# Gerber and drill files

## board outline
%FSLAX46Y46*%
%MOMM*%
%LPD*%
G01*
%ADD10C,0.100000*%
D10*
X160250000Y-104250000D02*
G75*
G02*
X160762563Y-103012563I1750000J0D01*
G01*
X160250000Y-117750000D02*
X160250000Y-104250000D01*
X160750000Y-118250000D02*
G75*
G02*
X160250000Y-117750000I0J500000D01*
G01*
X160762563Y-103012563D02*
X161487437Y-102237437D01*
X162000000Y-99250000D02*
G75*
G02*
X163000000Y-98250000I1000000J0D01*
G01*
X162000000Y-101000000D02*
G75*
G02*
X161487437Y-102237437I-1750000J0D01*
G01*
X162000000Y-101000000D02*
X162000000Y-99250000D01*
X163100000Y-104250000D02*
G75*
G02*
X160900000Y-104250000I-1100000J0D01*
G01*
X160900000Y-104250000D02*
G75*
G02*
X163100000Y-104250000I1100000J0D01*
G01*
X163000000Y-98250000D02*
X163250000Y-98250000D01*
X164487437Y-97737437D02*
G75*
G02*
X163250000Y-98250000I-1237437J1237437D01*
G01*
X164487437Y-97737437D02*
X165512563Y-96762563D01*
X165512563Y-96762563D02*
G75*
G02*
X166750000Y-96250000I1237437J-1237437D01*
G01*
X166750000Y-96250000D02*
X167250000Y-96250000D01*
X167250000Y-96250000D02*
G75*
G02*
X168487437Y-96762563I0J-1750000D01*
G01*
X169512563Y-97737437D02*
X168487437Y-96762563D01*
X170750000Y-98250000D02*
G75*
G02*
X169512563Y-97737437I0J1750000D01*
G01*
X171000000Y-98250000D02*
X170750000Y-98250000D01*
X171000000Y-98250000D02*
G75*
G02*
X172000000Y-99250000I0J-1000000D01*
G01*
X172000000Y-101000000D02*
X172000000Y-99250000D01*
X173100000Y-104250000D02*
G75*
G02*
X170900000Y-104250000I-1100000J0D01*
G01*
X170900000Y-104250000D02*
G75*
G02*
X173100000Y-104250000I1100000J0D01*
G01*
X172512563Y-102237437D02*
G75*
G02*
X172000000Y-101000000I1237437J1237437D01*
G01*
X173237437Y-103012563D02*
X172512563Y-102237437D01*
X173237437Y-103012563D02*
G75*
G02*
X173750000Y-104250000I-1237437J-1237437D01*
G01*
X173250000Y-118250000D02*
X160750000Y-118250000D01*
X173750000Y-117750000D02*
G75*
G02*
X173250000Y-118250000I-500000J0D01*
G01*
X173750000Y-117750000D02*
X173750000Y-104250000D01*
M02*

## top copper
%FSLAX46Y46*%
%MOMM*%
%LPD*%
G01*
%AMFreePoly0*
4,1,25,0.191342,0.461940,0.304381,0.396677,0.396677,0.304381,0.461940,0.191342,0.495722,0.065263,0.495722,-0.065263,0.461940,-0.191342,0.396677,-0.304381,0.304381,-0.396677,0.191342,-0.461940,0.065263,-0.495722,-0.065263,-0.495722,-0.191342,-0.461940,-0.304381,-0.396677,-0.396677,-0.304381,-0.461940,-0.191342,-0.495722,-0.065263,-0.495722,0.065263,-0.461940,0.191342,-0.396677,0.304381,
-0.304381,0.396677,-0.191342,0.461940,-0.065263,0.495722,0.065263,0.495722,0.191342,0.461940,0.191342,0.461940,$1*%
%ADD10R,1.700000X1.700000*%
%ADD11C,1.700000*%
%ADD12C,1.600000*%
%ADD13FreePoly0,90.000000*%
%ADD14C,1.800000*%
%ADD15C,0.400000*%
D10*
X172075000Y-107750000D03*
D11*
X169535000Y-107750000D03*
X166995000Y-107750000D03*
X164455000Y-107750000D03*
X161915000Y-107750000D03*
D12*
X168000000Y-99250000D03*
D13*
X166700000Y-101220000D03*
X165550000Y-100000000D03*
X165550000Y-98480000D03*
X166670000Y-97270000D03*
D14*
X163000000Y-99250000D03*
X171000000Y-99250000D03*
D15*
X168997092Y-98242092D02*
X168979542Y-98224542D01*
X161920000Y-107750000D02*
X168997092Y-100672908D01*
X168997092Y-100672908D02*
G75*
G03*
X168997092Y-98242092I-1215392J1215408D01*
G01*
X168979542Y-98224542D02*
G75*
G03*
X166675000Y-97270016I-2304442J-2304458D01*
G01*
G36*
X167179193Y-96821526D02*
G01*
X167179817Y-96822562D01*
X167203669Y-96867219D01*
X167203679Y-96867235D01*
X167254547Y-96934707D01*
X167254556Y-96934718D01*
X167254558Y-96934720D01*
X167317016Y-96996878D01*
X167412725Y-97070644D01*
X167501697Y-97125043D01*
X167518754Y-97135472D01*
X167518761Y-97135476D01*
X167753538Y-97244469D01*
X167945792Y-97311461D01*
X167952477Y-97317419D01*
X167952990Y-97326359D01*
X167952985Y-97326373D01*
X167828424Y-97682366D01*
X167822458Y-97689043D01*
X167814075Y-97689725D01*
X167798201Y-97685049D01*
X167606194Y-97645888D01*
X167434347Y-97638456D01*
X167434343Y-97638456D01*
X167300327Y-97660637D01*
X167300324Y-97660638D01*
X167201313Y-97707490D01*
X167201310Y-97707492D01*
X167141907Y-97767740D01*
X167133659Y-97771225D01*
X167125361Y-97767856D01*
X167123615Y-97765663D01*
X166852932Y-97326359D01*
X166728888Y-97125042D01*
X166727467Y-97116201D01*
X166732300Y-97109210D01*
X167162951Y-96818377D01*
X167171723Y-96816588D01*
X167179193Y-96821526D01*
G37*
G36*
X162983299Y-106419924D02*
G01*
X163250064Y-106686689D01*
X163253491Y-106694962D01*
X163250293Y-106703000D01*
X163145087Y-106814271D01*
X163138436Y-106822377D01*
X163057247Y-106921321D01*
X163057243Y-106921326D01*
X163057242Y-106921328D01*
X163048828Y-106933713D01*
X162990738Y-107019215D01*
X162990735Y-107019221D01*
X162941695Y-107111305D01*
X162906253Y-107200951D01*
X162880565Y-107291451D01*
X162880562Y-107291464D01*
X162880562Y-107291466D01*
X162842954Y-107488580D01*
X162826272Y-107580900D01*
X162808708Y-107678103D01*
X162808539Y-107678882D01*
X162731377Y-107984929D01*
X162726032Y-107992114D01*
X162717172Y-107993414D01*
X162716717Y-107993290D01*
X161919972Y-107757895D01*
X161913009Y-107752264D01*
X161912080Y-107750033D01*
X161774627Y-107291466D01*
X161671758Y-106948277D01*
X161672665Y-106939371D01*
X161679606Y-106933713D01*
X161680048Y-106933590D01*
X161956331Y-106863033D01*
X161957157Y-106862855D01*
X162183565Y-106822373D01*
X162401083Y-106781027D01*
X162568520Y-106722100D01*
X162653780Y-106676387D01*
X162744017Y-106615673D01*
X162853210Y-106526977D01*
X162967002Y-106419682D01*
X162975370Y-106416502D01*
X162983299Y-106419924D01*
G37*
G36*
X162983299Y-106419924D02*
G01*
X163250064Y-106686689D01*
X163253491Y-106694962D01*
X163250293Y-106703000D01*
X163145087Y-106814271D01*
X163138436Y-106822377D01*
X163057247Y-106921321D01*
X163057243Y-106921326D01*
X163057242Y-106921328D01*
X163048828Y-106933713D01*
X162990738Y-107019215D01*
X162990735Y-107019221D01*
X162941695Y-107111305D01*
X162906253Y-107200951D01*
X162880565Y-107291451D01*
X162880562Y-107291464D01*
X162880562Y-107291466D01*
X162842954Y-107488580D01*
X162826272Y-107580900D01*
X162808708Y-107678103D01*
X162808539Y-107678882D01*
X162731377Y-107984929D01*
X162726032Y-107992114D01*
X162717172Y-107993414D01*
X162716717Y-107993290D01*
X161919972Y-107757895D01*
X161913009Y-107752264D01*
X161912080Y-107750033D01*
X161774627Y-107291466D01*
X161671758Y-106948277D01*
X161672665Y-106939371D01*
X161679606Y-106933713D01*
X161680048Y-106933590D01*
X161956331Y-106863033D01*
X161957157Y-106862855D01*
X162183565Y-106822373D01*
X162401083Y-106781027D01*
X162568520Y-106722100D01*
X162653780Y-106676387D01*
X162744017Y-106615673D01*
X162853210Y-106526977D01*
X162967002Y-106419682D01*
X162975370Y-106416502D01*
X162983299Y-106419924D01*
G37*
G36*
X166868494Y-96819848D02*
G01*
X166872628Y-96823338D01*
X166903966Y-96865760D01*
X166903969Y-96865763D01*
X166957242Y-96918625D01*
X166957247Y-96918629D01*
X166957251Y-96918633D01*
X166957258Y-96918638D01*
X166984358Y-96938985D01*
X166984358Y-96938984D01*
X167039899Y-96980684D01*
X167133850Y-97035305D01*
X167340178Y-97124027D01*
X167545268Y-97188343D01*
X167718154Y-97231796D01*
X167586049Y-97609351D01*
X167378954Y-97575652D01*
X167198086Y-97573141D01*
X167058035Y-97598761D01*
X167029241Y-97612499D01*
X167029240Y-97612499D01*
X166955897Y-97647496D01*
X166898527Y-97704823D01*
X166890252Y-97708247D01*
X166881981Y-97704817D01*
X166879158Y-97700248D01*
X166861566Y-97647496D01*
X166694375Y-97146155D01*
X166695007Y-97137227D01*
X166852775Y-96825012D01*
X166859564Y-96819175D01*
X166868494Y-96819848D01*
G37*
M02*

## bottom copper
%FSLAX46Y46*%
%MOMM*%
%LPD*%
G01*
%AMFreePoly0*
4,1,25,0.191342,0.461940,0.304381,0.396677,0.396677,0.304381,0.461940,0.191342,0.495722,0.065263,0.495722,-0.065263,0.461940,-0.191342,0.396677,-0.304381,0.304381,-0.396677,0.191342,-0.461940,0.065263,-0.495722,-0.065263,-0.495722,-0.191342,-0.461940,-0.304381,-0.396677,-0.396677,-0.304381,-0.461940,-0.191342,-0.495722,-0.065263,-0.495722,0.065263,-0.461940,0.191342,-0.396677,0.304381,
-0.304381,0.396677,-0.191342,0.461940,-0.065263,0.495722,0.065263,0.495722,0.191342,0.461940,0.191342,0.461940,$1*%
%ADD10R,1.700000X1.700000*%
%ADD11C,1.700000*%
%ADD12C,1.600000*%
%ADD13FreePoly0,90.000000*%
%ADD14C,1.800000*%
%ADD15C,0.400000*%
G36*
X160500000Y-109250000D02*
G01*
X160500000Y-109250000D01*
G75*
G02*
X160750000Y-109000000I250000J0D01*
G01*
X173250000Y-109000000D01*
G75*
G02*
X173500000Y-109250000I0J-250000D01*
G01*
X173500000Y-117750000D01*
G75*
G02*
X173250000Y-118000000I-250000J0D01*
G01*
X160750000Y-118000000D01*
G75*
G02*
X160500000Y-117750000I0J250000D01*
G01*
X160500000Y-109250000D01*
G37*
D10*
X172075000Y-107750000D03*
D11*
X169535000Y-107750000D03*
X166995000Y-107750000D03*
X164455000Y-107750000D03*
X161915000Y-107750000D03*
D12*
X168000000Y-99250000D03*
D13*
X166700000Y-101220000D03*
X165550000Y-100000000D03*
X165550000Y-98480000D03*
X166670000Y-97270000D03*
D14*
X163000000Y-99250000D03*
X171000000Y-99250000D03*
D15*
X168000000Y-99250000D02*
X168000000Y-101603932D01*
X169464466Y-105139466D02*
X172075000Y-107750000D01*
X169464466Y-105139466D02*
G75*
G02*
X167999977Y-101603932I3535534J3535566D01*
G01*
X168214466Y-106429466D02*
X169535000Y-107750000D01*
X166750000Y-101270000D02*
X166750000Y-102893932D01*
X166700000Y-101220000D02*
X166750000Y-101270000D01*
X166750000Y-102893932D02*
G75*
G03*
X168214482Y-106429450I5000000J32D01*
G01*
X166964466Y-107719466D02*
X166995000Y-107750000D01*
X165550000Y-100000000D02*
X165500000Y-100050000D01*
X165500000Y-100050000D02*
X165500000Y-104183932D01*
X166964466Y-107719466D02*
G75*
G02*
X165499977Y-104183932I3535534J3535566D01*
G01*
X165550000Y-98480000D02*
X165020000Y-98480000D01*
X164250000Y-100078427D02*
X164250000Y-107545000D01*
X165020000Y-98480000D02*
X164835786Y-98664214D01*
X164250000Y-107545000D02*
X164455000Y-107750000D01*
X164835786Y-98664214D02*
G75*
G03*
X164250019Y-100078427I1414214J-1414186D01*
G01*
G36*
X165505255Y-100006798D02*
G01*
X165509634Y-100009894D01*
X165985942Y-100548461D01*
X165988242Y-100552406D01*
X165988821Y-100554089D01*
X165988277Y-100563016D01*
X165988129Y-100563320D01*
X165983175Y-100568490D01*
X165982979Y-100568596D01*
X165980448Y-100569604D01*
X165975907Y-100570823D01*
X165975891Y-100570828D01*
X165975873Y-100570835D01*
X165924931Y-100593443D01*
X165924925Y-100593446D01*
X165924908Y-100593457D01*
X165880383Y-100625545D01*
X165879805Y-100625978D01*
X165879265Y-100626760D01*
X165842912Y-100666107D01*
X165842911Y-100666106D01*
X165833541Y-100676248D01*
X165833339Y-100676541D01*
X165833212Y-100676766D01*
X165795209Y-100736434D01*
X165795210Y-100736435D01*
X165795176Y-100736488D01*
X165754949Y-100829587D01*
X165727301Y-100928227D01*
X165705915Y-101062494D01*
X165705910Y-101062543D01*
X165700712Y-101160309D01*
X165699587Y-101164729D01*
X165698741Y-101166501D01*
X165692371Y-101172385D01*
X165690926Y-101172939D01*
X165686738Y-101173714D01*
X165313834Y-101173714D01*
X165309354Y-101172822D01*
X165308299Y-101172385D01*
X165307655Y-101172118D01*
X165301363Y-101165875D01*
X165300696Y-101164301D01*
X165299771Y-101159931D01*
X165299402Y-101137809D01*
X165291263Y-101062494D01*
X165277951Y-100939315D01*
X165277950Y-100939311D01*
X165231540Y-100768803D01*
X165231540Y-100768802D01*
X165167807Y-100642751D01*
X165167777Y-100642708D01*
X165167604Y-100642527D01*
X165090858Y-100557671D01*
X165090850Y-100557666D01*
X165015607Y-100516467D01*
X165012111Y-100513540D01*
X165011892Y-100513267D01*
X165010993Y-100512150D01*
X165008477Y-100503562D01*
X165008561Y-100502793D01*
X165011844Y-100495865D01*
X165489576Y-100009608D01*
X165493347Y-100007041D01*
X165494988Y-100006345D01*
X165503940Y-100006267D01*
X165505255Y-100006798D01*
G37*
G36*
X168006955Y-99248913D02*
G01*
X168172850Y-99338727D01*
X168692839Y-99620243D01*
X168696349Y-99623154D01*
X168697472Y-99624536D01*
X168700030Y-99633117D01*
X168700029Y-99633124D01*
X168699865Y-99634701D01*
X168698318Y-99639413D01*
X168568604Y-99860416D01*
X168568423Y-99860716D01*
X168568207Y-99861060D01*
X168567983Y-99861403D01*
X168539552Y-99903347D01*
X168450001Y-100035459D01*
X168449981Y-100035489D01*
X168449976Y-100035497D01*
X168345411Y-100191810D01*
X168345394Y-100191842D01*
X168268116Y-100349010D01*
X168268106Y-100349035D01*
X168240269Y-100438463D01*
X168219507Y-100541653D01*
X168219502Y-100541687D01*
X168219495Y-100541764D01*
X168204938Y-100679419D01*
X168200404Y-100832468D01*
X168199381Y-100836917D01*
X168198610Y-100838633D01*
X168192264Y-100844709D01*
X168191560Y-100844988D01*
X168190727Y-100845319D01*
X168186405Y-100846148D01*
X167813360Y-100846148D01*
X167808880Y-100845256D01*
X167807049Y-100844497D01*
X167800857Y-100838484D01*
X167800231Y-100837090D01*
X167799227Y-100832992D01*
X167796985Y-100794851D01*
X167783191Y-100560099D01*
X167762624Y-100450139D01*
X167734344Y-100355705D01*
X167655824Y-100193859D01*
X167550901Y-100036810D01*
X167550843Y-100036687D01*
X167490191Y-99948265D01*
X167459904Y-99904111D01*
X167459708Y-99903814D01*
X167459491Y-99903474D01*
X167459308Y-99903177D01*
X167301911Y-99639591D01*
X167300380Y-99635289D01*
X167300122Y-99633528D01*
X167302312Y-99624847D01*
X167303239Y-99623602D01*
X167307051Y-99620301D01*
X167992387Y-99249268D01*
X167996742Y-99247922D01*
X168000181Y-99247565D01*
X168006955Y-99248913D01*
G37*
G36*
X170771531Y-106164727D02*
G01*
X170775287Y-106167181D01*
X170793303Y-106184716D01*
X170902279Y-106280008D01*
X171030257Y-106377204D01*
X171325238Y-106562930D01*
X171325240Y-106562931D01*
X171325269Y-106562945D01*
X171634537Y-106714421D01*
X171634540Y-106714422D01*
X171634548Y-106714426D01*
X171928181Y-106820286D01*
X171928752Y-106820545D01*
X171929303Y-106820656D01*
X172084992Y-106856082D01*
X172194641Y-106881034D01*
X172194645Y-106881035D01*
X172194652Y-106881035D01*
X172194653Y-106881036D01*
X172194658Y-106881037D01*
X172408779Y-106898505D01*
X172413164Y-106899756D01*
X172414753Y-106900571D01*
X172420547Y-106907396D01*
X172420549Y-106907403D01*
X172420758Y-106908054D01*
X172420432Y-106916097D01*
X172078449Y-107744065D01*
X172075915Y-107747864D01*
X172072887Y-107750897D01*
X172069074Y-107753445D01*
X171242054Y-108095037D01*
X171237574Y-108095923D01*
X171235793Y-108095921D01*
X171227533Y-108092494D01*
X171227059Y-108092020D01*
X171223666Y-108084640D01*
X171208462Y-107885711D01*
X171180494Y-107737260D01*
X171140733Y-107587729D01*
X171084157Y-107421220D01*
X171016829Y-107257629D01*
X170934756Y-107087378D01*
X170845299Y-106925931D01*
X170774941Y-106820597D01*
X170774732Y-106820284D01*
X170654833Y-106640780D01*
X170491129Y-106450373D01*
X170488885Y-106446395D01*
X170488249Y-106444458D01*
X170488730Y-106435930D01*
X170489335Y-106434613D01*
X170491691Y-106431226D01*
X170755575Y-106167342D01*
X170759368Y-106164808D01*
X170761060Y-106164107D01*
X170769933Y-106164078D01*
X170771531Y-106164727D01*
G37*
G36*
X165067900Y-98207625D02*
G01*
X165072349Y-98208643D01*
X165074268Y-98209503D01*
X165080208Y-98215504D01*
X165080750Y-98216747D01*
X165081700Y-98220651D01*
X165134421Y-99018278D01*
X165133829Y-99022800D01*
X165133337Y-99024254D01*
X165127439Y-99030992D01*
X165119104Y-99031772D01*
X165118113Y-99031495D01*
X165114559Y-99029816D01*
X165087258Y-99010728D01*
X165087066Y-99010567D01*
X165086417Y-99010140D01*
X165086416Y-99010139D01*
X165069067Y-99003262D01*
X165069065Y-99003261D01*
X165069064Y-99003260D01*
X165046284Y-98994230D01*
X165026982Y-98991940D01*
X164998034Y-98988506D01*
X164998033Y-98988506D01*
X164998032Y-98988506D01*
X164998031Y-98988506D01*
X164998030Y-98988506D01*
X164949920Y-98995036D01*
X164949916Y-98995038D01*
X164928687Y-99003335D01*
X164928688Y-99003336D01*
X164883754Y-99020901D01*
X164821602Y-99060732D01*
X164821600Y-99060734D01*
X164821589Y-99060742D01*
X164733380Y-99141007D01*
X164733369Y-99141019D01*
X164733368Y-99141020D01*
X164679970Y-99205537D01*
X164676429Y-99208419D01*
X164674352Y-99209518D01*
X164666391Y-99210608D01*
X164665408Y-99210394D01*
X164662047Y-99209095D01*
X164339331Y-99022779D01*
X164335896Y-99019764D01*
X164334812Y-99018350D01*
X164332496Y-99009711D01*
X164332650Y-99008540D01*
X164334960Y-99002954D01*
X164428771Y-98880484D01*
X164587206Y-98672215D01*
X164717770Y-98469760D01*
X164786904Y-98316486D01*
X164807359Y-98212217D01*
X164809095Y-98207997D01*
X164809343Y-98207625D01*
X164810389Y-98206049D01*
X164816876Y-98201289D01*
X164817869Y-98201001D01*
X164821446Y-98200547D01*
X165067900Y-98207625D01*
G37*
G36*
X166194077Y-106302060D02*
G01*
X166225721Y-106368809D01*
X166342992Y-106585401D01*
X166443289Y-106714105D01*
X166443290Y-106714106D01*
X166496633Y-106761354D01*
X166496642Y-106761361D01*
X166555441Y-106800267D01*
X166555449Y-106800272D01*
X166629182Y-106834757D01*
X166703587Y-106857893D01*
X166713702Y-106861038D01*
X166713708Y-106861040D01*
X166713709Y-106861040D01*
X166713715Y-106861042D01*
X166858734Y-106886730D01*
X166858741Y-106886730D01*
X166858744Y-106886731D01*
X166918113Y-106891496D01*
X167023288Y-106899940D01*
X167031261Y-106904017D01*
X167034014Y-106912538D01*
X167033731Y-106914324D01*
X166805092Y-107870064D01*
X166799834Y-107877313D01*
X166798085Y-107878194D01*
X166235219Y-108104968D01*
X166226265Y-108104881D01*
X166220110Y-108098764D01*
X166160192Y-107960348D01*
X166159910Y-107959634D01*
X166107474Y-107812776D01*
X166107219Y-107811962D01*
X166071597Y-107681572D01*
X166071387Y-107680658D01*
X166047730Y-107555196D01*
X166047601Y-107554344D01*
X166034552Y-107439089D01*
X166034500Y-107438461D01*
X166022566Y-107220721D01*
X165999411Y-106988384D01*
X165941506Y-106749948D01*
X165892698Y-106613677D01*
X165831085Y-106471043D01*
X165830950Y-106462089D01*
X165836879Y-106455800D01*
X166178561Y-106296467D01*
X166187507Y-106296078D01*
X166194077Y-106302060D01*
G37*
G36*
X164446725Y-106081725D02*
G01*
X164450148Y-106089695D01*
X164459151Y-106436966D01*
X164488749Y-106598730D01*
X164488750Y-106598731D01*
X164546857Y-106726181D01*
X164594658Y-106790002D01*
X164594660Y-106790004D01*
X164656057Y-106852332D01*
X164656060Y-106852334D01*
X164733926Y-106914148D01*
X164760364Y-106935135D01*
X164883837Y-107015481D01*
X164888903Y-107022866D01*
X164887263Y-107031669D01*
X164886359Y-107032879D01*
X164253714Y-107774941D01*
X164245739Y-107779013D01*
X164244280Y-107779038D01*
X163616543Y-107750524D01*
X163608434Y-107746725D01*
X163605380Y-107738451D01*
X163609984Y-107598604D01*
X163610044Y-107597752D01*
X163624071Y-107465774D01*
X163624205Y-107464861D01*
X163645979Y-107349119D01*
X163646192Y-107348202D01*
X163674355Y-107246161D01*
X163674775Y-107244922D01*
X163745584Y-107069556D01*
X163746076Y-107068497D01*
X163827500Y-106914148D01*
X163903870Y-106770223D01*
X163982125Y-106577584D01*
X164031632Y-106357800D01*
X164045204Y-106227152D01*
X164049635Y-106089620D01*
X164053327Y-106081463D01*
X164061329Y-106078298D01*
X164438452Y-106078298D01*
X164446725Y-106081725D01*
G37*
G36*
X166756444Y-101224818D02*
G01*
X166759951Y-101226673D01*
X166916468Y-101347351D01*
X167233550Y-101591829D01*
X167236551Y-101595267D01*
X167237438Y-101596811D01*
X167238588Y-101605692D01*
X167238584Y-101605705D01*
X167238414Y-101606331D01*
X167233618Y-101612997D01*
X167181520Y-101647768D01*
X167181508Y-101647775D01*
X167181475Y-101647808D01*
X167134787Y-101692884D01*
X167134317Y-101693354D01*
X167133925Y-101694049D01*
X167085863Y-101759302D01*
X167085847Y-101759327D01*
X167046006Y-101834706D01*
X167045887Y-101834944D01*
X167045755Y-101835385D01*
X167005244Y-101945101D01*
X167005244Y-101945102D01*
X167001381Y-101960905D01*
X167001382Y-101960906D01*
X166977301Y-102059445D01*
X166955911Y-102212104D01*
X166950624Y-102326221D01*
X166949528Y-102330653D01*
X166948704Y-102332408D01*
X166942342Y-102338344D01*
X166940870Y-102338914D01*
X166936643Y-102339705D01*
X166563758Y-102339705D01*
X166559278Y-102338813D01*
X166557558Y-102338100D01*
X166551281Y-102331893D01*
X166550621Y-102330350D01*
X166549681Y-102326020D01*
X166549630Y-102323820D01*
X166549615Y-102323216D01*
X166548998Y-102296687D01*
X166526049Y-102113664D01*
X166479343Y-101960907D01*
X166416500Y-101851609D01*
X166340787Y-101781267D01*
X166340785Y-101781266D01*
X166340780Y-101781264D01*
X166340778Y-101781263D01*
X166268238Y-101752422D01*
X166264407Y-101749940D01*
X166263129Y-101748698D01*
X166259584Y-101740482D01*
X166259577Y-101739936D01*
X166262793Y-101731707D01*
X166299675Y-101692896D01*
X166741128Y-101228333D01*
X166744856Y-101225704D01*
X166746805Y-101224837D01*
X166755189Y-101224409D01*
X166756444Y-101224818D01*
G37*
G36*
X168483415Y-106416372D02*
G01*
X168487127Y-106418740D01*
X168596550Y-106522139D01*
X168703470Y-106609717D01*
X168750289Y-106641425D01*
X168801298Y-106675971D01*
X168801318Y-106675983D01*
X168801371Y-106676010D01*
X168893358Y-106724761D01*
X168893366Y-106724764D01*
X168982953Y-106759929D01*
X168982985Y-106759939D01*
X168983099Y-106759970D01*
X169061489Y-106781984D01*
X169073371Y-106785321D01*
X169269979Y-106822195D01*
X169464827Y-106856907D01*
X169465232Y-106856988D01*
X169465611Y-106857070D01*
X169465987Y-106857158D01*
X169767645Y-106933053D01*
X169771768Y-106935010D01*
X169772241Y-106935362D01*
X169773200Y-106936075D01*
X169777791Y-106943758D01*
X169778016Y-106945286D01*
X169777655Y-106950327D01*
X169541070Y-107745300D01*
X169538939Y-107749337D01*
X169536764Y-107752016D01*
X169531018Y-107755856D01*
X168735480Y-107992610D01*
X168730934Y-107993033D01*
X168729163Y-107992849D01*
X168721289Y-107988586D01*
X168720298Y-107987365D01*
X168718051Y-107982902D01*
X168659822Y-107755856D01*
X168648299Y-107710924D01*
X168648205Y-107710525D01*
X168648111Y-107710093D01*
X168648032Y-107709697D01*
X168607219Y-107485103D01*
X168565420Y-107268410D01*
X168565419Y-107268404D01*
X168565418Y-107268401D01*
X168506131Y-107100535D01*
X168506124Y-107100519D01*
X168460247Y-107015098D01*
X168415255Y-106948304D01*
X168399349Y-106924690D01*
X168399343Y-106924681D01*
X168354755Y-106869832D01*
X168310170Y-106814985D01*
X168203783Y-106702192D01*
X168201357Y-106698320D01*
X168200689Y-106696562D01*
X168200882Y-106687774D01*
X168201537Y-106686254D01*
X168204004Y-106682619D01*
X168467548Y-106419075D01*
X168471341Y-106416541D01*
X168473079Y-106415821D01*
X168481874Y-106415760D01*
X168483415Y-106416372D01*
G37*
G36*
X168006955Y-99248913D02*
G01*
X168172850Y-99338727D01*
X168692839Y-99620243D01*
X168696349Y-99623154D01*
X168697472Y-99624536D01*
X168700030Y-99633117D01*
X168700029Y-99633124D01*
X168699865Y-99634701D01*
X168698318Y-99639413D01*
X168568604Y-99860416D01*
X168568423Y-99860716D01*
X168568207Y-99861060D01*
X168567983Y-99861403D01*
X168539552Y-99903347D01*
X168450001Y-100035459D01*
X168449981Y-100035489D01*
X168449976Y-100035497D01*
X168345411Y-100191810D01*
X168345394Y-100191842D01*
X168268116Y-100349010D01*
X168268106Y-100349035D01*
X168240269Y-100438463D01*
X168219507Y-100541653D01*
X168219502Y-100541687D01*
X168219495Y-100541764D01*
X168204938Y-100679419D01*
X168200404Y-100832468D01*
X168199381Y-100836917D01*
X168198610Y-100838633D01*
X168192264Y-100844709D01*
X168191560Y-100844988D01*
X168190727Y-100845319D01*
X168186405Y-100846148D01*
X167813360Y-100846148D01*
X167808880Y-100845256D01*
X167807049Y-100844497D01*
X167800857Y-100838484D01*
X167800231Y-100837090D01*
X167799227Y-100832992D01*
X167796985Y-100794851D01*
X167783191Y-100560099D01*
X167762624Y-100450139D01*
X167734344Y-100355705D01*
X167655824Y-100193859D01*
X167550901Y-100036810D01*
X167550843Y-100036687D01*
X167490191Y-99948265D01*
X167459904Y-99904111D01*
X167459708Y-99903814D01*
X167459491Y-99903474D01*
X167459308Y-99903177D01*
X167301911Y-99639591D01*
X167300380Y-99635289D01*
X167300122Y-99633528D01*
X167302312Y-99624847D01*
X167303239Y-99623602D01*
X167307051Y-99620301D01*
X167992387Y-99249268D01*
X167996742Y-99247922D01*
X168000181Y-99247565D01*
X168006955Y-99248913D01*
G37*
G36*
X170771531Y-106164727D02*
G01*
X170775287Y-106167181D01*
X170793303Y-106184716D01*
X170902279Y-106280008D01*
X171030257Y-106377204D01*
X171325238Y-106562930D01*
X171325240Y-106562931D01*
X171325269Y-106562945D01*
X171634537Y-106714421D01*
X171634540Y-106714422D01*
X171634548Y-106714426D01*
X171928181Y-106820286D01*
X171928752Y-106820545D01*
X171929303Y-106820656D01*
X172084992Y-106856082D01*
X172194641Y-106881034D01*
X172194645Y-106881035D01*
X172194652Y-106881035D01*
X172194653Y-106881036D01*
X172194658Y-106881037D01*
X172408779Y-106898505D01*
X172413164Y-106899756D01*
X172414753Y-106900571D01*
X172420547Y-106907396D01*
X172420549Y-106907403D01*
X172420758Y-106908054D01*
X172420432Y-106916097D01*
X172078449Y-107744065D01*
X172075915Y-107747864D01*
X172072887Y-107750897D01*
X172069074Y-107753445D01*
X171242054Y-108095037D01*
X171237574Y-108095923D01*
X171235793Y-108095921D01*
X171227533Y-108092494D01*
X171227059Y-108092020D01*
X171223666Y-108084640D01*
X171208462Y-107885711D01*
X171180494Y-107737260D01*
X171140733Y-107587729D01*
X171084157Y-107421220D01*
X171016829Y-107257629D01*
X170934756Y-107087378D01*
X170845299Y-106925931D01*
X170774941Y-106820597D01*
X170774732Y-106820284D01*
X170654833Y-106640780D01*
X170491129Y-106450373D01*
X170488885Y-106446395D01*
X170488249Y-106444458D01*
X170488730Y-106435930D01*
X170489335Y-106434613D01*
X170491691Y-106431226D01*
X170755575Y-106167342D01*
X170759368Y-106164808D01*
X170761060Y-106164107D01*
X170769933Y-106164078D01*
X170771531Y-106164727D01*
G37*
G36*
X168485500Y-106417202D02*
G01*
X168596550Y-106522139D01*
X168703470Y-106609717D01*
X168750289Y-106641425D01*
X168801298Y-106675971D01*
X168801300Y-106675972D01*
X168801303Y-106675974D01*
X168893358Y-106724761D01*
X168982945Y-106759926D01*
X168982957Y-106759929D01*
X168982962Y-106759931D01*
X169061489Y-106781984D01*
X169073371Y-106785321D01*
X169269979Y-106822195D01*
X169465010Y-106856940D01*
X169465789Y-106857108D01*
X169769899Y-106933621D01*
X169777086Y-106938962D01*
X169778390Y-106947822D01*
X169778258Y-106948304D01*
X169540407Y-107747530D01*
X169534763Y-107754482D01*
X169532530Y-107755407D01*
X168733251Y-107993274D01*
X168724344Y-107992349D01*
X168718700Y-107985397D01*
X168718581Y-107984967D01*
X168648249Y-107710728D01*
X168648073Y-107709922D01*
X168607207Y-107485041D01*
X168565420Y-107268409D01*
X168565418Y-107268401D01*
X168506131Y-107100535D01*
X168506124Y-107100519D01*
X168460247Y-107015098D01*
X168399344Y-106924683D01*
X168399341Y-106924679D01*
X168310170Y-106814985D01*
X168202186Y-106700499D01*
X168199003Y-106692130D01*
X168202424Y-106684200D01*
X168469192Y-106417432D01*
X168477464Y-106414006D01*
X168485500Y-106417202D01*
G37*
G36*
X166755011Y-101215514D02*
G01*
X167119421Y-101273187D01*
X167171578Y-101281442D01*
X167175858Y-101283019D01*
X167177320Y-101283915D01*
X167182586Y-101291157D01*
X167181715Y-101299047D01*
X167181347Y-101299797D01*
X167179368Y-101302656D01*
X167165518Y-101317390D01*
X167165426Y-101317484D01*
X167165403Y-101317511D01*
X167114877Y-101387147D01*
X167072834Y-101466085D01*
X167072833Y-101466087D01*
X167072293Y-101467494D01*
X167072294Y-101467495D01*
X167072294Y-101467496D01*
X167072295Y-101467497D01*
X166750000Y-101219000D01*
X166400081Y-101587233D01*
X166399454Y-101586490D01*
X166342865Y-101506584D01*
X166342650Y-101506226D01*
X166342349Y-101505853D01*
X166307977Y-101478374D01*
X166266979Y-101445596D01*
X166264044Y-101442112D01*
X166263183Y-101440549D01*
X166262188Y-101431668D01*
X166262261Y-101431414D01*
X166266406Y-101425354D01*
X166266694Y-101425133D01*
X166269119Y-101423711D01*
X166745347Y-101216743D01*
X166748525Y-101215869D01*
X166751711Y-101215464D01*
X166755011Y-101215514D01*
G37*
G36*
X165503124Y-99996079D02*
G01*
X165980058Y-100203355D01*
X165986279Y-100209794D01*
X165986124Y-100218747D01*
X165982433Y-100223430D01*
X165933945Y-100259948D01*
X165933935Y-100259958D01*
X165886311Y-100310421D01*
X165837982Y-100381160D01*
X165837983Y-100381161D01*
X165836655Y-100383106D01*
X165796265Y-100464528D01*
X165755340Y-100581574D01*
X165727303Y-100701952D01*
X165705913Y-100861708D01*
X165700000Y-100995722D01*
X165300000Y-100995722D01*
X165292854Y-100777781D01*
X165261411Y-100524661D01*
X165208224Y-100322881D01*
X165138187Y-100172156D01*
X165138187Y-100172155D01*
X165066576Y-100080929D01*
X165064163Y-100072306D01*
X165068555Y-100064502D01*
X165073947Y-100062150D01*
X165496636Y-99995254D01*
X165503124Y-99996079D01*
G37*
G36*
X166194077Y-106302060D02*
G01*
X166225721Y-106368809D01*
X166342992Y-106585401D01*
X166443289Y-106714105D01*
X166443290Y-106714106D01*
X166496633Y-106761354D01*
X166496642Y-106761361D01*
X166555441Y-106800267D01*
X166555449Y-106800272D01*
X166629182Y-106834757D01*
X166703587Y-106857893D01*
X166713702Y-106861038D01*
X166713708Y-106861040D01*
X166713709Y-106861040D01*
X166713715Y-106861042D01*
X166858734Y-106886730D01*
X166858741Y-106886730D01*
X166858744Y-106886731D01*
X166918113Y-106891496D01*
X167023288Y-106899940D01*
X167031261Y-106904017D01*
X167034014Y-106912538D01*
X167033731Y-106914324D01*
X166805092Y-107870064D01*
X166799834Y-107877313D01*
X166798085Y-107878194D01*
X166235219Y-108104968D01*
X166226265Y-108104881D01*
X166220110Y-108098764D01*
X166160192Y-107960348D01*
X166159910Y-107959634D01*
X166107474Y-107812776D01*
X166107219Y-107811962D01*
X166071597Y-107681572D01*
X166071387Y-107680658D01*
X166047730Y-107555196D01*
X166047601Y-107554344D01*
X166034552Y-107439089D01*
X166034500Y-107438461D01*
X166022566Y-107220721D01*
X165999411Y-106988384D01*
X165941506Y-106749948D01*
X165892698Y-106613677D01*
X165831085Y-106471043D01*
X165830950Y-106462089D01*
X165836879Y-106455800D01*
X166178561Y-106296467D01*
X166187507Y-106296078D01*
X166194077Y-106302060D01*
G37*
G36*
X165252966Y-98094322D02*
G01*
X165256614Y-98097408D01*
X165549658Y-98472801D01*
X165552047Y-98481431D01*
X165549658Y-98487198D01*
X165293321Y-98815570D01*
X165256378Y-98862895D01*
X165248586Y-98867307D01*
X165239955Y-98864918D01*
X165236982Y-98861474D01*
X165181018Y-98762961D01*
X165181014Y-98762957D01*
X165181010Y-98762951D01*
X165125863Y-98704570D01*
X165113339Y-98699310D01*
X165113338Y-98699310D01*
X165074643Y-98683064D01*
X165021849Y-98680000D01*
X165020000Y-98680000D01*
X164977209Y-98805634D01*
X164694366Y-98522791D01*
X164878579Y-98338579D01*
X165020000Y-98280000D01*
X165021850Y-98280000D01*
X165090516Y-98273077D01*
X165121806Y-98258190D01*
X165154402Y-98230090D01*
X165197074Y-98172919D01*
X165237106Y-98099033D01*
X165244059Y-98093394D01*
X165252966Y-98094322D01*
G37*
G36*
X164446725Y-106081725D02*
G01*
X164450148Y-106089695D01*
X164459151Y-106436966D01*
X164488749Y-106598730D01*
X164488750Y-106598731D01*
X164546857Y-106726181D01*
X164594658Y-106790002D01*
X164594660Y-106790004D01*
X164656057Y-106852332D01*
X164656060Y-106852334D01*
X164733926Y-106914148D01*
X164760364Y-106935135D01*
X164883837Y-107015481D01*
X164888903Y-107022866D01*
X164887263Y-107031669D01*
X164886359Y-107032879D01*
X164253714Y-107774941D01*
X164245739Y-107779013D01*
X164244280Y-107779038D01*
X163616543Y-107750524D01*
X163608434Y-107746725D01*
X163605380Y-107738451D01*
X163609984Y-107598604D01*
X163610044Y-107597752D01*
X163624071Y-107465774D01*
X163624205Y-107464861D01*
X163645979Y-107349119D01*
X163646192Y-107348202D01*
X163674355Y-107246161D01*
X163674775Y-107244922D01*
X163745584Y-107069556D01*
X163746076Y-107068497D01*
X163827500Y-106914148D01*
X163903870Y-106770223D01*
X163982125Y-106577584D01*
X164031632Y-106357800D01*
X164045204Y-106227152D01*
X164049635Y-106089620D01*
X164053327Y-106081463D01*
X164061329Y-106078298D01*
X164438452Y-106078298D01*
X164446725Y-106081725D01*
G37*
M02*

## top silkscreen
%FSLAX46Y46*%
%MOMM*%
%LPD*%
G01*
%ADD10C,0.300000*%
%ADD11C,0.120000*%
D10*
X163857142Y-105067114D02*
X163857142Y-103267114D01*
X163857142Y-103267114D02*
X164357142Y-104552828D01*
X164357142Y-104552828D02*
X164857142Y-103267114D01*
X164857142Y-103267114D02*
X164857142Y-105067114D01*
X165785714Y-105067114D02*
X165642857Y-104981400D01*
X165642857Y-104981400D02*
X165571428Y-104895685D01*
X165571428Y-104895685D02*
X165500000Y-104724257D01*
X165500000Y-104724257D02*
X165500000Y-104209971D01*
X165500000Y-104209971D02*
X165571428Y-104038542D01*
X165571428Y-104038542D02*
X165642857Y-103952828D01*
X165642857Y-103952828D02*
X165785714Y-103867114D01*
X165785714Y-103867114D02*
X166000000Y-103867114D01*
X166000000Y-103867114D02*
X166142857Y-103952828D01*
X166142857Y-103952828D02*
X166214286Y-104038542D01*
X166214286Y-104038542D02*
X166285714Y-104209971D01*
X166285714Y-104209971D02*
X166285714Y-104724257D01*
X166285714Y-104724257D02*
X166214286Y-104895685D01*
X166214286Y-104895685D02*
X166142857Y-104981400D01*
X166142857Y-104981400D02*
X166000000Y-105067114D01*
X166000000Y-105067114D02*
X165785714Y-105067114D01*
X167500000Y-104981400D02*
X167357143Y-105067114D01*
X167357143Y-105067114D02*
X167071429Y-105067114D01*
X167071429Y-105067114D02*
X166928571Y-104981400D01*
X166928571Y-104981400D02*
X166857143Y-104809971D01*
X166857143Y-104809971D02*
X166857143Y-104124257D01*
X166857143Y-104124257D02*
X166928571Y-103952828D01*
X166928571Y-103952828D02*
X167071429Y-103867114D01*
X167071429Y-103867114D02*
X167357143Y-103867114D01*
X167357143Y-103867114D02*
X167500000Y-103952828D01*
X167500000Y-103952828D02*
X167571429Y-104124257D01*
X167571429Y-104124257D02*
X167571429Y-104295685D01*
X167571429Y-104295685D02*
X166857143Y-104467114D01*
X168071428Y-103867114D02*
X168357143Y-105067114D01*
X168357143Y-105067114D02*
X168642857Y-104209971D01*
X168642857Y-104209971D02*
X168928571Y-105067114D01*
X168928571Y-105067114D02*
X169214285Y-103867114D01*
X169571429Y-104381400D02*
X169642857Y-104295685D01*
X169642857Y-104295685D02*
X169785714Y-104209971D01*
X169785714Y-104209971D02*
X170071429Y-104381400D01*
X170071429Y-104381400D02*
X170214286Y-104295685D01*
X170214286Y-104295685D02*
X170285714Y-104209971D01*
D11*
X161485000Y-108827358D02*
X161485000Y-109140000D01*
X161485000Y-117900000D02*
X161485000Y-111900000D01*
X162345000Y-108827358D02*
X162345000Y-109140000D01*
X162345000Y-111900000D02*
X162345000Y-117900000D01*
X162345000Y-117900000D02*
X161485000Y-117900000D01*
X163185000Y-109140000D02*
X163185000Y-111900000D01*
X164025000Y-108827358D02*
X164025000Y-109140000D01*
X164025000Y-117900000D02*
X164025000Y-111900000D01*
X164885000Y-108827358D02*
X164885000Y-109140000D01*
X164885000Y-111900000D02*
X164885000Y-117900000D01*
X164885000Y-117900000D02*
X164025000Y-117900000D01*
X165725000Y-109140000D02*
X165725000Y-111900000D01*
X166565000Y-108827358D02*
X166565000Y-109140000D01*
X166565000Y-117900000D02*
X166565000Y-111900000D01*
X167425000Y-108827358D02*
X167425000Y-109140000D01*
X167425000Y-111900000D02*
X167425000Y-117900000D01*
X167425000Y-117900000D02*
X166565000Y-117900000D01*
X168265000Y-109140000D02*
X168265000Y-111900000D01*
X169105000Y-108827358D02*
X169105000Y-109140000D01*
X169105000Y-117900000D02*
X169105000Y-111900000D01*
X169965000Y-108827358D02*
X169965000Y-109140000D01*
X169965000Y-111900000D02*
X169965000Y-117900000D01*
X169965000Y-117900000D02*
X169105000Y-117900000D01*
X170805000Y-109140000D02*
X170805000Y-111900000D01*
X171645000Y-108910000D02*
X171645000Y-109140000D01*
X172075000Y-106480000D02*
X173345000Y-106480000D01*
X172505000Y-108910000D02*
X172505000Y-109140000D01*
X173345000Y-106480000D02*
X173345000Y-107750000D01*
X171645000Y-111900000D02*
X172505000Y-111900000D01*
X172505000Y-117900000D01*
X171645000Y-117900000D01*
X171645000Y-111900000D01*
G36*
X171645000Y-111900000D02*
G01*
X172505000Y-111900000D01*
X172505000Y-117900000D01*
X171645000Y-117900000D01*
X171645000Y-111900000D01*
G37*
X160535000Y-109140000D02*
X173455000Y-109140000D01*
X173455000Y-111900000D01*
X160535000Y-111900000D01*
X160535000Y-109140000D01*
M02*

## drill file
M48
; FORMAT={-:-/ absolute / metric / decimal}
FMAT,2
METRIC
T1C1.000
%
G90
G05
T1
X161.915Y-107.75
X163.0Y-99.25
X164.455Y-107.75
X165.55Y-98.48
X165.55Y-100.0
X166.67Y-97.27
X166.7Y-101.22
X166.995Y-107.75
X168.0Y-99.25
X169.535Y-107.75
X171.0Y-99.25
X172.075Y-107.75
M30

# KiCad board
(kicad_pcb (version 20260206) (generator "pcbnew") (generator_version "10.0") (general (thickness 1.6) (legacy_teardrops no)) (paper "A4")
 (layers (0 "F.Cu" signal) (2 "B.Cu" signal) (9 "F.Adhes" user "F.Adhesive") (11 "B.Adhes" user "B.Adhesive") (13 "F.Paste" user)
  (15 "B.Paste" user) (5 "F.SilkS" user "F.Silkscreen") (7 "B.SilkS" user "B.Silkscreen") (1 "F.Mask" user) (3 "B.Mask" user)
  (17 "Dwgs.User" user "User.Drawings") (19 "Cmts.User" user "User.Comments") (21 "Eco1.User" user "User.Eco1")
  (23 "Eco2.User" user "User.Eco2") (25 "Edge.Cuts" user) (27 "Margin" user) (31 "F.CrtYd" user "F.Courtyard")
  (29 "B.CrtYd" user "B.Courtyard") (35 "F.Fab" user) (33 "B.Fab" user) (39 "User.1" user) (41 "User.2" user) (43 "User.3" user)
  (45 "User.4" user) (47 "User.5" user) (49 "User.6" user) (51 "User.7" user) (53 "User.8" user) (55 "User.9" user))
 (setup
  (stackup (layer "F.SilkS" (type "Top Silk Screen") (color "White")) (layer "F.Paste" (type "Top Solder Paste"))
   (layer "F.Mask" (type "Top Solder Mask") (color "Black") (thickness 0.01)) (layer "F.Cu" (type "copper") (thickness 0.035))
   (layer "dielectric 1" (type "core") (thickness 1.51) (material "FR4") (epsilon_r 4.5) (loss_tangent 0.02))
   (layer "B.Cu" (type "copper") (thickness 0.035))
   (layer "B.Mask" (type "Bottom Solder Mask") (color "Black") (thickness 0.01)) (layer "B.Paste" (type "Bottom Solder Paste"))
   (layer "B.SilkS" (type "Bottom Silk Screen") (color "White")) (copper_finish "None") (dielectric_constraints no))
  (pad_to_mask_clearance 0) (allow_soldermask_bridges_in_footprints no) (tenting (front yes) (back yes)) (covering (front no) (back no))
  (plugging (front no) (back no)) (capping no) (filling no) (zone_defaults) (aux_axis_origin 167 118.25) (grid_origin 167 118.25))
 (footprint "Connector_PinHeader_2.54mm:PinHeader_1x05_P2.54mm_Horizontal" (layer "F.Cu") (at 172.075 107.75 -90)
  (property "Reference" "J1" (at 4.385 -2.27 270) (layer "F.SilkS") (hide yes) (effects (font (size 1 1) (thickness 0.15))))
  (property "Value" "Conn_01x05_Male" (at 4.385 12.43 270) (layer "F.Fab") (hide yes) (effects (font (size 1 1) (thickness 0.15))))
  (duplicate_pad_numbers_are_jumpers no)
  (fp_line (start 1.077358 10.59) (end 1.39 10.59) (stroke (width 0.12) (type solid)) (layer "F.SilkS"))
  (fp_line (start 10.15 10.59) (end 4.15 10.59) (stroke (width 0.12) (type solid)) (layer "F.SilkS"))
  (fp_line (start 1.077358 9.73) (end 1.39 9.73) (stroke (width 0.12) (type solid)) (layer "F.SilkS"))
  (fp_line (start 4.15 9.73) (end 10.15 9.73) (stroke (width 0.12) (type solid)) (layer "F.SilkS"))
  (fp_line (start 10.15 9.73) (end 10.15 10.59) (stroke (width 0.12) (type solid)) (layer "F.SilkS"))
  (fp_line (start 1.39 8.89) (end 4.15 8.89) (stroke (width 0.12) (type solid)) (layer "F.SilkS"))
  (fp_line (start 1.077358 8.05) (end 1.39 8.05) (stroke (width 0.12) (type solid)) (layer "F.SilkS"))
  (fp_line (start 10.15 8.05) (end 4.15 8.05) (stroke (width 0.12) (type solid)) (layer "F.SilkS"))
  (fp_line (start 1.077358 7.19) (end 1.39 7.19) (stroke (width 0.12) (type solid)) (layer "F.SilkS"))
  (fp_line (start 4.15 7.19) (end 10.15 7.19) (stroke (width 0.12) (type solid)) (layer "F.SilkS"))
  (fp_line (start 10.15 7.19) (end 10.15 8.05) (stroke (width 0.12) (type solid)) (layer "F.SilkS"))
  (fp_line (start 1.39 6.35) (end 4.15 6.35) (stroke (width 0.12) (type solid)) (layer "F.SilkS"))
  (fp_line (start 1.077358 5.51) (end 1.39 5.51) (stroke (width 0.12) (type solid)) (layer "F.SilkS"))
  (fp_line (start 10.15 5.51) (end 4.15 5.51) (stroke (width 0.12) (type solid)) (layer "F.SilkS"))
  (fp_line (start 1.077358 4.65) (end 1.39 4.65) (stroke (width 0.12) (type solid)) (layer "F.SilkS"))
  (fp_line (start 4.15 4.65) (end 10.15 4.65) (stroke (width 0.12) (type solid)) (layer "F.SilkS"))
  (fp_line (start 10.15 4.65) (end 10.15 5.51) (stroke (width 0.12) (type solid)) (layer "F.SilkS"))
  (fp_line (start 1.39 3.81) (end 4.15 3.81) (stroke (width 0.12) (type solid)) (layer "F.SilkS"))
  (fp_line (start 1.077358 2.97) (end 1.39 2.97) (stroke (width 0.12) (type solid)) (layer "F.SilkS"))
  (fp_line (start 10.15 2.97) (end 4.15 2.97) (stroke (width 0.12) (type solid)) (layer "F.SilkS"))
  (fp_line (start 1.077358 2.11) (end 1.39 2.11) (stroke (width 0.12) (type solid)) (layer "F.SilkS"))
  (fp_line (start 4.15 2.11) (end 10.15 2.11) (stroke (width 0.12) (type solid)) (layer "F.SilkS"))
  (fp_line (start 10.15 2.11) (end 10.15 2.97) (stroke (width 0.12) (type solid)) (layer "F.SilkS"))
  (fp_line (start 1.39 1.27) (end 4.15 1.27) (stroke (width 0.12) (type solid)) (layer "F.SilkS"))
  (fp_line (start 1.16 0.43) (end 1.39 0.43) (stroke (width 0.12) (type solid)) (layer "F.SilkS"))
  (fp_line (start -1.27 0) (end -1.27 -1.27) (stroke (width 0.12) (type solid)) (layer "F.SilkS"))
  (fp_line (start 1.16 -0.43) (end 1.39 -0.43) (stroke (width 0.12) (type solid)) (layer "F.SilkS"))
  (fp_line (start -1.27 -1.27) (end 0 -1.27) (stroke (width 0.12) (type solid)) (layer "F.SilkS"))
  (fp_rect (start 4.15 -0.43) (end 10.15 0.43) (stroke (width 0.12) (type solid)) (fill yes) (layer "F.SilkS"))
  (fp_rect (start 1.39 -1.38) (end 4.15 11.54) (stroke (width 0.12) (type solid)) (fill no) (layer "F.SilkS"))
  (pad "1" thru_hole rect (at 0 0 270) (size 1.7 1.7) (drill 1) (layers "*.Cu" "*.Mask") (remove_unused_layers no) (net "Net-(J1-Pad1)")
   (teardrops (best_length_ratio 0.5) (max_length 1) (best_width_ratio 1) (max_width 2) (curved_edges yes) (filter_ratio 0.9) (enabled yes)
    (allow_two_segments yes) (prefer_zone_connections yes)))
  (pad "2" thru_hole circle (at 0 2.54 270) (size 1.7 1.7) (drill 1) (layers "*.Cu" "*.Mask") (remove_unused_layers no)
   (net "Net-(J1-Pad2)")
   (teardrops (best_length_ratio 0.5) (max_length 1) (best_width_ratio 1) (max_width 2) (curved_edges yes) (filter_ratio 0.9) (enabled yes)
    (allow_two_segments yes) (prefer_zone_connections yes)))
  (pad "3" thru_hole circle (at 0 5.08 270) (size 1.7 1.7) (drill 1) (layers "*.Cu" "*.Mask") (remove_unused_layers no)
   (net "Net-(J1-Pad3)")
   (teardrops (best_length_ratio 0.5) (max_length 1) (best_width_ratio 1) (max_width 2) (curved_edges yes) (filter_ratio 0.9) (enabled yes)
    (allow_two_segments yes) (prefer_zone_connections yes)))
  (pad "4" thru_hole circle (at 0 7.62 270) (size 1.7 1.7) (drill 1) (layers "*.Cu" "*.Mask") (remove_unused_layers no)
   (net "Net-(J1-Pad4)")
   (teardrops (best_length_ratio 0.5) (max_length 1) (best_width_ratio 1) (max_width 2) (curved_edges yes) (filter_ratio 0.9) (enabled yes)
    (allow_two_segments yes) (prefer_zone_connections yes)))
  (pad "5" thru_hole circle (at 0 10.16 270) (size 1.7 1.7) (drill 1) (layers "*.Cu" "*.Mask") (remove_unused_layers no)
   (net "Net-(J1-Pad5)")
   (teardrops (best_length_ratio 0.5) (max_length 1) (best_width_ratio 1) (max_width 2) (curved_edges yes) (filter_ratio 0.9) (enabled yes)
    (allow_two_segments yes) (prefer_zone_connections yes))))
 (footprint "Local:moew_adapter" (layer "F.Cu") (at 167 99.25 90)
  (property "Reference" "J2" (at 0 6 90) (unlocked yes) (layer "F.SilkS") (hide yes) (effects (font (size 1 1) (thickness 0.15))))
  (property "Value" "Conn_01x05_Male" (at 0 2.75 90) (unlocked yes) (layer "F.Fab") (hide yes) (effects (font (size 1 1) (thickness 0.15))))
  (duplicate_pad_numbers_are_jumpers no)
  (pad "1" thru_hole circle (at 0 1 90) (size 1.6 1.6) (drill 1) (layers "*.Cu" "F.Mask") (remove_unused_layers no) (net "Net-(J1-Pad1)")
   (teardrops (best_length_ratio 0.5) (max_length 1) (best_width_ratio 1) (max_width 2) (curved_edges yes) (filter_ratio 0.9) (enabled yes)
    (allow_two_segments yes) (prefer_zone_connections yes)))
  (pad "2" thru_hole custom (at -1.97 -0.3 90) (size 1 1) (drill 1) (layers "*.Cu" "F.Mask") (remove_unused_layers no) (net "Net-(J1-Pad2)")
   (thermal_bridge_angle 90) (options (clearance outline) (anchor circle)) (primitives)
   (teardrops (best_length_ratio 0.5) (max_length 1) (best_width_ratio 1) (max_width 2) (curved_edges yes) (filter_ratio 0.9) (enabled yes)
    (allow_two_segments yes) (prefer_zone_connections yes)))
  (pad "3" thru_hole custom (at -0.75 -1.45 90) (size 1 1) (drill 1) (layers "*.Cu" "F.Mask") (remove_unused_layers no)
   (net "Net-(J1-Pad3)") (thermal_bridge_angle 90) (options (clearance outline) (anchor circle)) (primitives)
   (teardrops (best_length_ratio 0.5) (max_length 1) (best_width_ratio 1) (max_width 2) (curved_edges yes) (filter_ratio 0.9) (enabled yes)
    (allow_two_segments yes) (prefer_zone_connections yes)))
  (pad "4" thru_hole custom (at 0.77 -1.45 90) (size 1 1) (drill 1) (layers "*.Cu" "F.Mask") (remove_unused_layers no) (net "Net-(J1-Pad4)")
   (thermal_bridge_angle 90) (options (clearance outline) (anchor circle)) (primitives)
   (teardrops (best_length_ratio 0.5) (max_length 1) (best_width_ratio 1) (max_width 2) (curved_edges yes) (filter_ratio 0.9) (enabled yes)
    (allow_two_segments yes) (prefer_zone_connections yes)))
  (pad "5" thru_hole custom (at 1.98 -0.33 90) (size 1 1) (drill 1) (layers "*.Cu" "F.Mask") (remove_unused_layers no) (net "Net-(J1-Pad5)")
   (thermal_bridge_angle 90) (options (clearance outline) (anchor circle)) (primitives)
   (teardrops (best_length_ratio 0.5) (max_length 1) (best_width_ratio 1) (max_width 2) (curved_edges yes) (filter_ratio 0.9) (enabled yes)
    (allow_two_segments yes) (prefer_zone_connections yes)))
  (pad "NC" thru_hole circle (at 0 -4 90) (size 1.8 1.8) (drill 1) (layers "*.Cu" "*.Mask") (remove_unused_layers no)
   (solder_mask_margin -0.1))
  (pad "NC" thru_hole circle (at 0 4 90) (size 1.8 1.8) (drill 1) (layers "*.Cu" "*.Mask") (remove_unused_layers no)
   (solder_mask_margin -0.1)))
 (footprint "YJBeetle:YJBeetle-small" (layer "B.Cu") (at 167 116.5 180)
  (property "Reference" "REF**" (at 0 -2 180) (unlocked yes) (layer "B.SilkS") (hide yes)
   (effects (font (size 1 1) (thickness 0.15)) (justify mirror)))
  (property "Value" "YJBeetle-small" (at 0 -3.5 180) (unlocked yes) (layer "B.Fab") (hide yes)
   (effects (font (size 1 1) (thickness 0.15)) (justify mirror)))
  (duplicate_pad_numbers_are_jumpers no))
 (gr_rect (start 160.5 109) (end 173.5 118) (radius 0.25) (stroke (width 0) (type solid)) (fill yes) (layer "B.Cu"))
 (gr_arc (start 160.25 104.25) (mid 160.383211 103.580304) (end 160.762563 103.012563) (stroke (width 0.1) (type default))
  (layer "Edge.Cuts"))
 (gr_line (start 160.25 117.75) (end 160.25 104.25) (stroke (width 0.1) (type default)) (layer "Edge.Cuts"))
 (gr_arc (start 160.75 118.25) (mid 160.396447 118.103553) (end 160.25 117.75) (stroke (width 0.1) (type default)) (layer "Edge.Cuts"))
 (gr_line (start 160.762563 103.012563) (end 161.487437 102.237437) (stroke (width 0.1) (type default)) (layer "Edge.Cuts"))
 (gr_arc (start 162 99.25) (mid 162.292893 98.542893) (end 163 98.25) (stroke (width 0.1) (type default)) (layer "Edge.Cuts"))
 (gr_arc (start 162 101) (mid 161.866789 101.669696) (end 161.487437 102.237437) (stroke (width 0.1) (type default)) (layer "Edge.Cuts"))
 (gr_line (start 162 101) (end 162 99.25) (stroke (width 0.1) (type default)) (layer "Edge.Cuts"))
 (gr_circle (center 162 104.25) (end 163.1 104.25) (stroke (width 0.1) (type solid)) (fill no) (layer "Edge.Cuts"))
 (gr_line (start 163 98.25) (end 163.25 98.25) (stroke (width 0.1) (type default)) (layer "Edge.Cuts"))
 (gr_arc (start 164.487437 97.737437) (mid 163.919696 98.116789) (end 163.25 98.25) (stroke (width 0.1) (type default)) (layer "Edge.Cuts"))
 (gr_line (start 164.487437 97.737437) (end 165.512563 96.762563) (stroke (width 0.1) (type default)) (layer "Edge.Cuts"))
 (gr_arc (start 165.512563 96.762563) (mid 166.080304 96.383211) (end 166.75 96.25) (stroke (width 0.1) (type default)) (layer "Edge.Cuts"))
 (gr_line (start 166.75 96.25) (end 167.25 96.25) (stroke (width 0.1) (type default)) (layer "Edge.Cuts"))
 (gr_arc (start 167.25 96.25) (mid 167.919696 96.383211) (end 168.487437 96.762563) (stroke (width 0.1) (type default)) (layer "Edge.Cuts"))
 (gr_line (start 169.512563 97.737437) (end 168.487437 96.762563) (stroke (width 0.1) (type default)) (layer "Edge.Cuts"))
 (gr_arc (start 170.75 98.25) (mid 170.080304 98.116789) (end 169.512563 97.737437) (stroke (width 0.1) (type default)) (layer "Edge.Cuts"))
 (gr_line (start 171 98.25) (end 170.75 98.25) (stroke (width 0.1) (type default)) (layer "Edge.Cuts"))
 (gr_arc (start 171 98.25) (mid 171.707107 98.542893) (end 172 99.25) (stroke (width 0.1) (type default)) (layer "Edge.Cuts"))
 (gr_line (start 172 101) (end 172 99.25) (stroke (width 0.1) (type default)) (layer "Edge.Cuts"))
 (gr_circle (center 172 104.25) (end 173.1 104.25) (stroke (width 0.1) (type solid)) (fill no) (layer "Edge.Cuts"))
 (gr_arc (start 172.512563 102.237437) (mid 172.133211 101.669696) (end 172 101) (stroke (width 0.1) (type default)) (layer "Edge.Cuts"))
 (gr_line (start 173.237437 103.012563) (end 172.512563 102.237437) (stroke (width 0.1) (type default)) (layer "Edge.Cuts"))
 (gr_arc (start 173.237437 103.012563) (mid 173.616789 103.580304) (end 173.75 104.25) (stroke (width 0.1) (type default))
  (layer "Edge.Cuts"))
 (gr_line (start 173.25 118.25) (end 160.75 118.25) (stroke (width 0.1) (type default)) (layer "Edge.Cuts"))
 (gr_arc (start 173.75 117.75) (mid 173.603553 118.103553) (end 173.25 118.25) (stroke (width 0.1) (type default)) (layer "Edge.Cuts"))
 (gr_line (start 173.75 117.75) (end 173.75 104.25) (stroke (width 0.1) (type default)) (layer "Edge.Cuts"))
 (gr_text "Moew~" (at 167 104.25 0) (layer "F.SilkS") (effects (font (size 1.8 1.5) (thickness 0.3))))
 (segment (start 168 99.25) (end 168 101.603932) (width 0.4) (layer "B.Cu") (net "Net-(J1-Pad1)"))
 (segment (start 169.464466 105.139466) (end 172.075 107.75) (width 0.4) (layer "B.Cu") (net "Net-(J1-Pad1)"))
 (arc (start 169.464466 105.139466) (mid 168.380602 103.517349) (end 168 101.603932) (width 0.4) (layer "B.Cu") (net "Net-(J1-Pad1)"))
 (segment (start 168.214466 106.429466) (end 169.535 107.75) (width 0.4) (layer "B.Cu") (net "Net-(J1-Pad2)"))
 (segment (start 166.75 101.27) (end 166.75 102.893932) (width 0.4) (layer "B.Cu") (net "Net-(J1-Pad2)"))
 (segment (start 166.7 101.22) (end 166.75 101.27) (width 0.4) (layer "B.Cu") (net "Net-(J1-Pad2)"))
 (arc (start 166.75 102.893932) (mid 167.130602 104.807349) (end 168.214466 106.429466) (width 0.4) (layer "B.Cu") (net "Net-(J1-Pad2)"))
 (segment (start 166.964466 107.719466) (end 166.995 107.75) (width 0.4) (layer "B.Cu") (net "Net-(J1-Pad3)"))
 (segment (start 165.55 100) (end 165.5 100.05) (width 0.4) (layer "B.Cu") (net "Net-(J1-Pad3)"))
 (segment (start 165.5 100.05) (end 165.5 104.183932) (width 0.4) (layer "B.Cu") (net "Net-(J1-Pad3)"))
 (arc (start 166.964466 107.719466) (mid 165.880602 106.097349) (end 165.5 104.183932) (width 0.4) (layer "B.Cu") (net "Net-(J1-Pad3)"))
 (segment (start 165.55 98.48) (end 165.02 98.48) (width 0.4) (layer "B.Cu") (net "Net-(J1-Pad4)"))
 (segment (start 164.25 100.078427) (end 164.25 107.545) (width 0.4) (layer "B.Cu") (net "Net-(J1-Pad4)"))
 (segment (start 165.02 98.48) (end 164.835786 98.664214) (width 0.4) (layer "B.Cu") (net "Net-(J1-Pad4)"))
 (segment (start 164.25 107.545) (end 164.455 107.75) (width 0.4) (layer "B.Cu") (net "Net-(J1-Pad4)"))
 (arc (start 164.835786 98.664214) (mid 164.402241 99.31306) (end 164.25 100.078427) (width 0.4) (layer "B.Cu") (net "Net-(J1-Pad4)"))
 (segment (start 168.997092 98.242092) (end 168.979542 98.224542) (width 0.4) (layer "F.Cu") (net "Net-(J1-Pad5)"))
 (segment (start 161.92 107.75) (end 168.997092 100.672908) (width 0.4) (layer "F.Cu") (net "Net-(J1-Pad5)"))
 (arc (start 168.997092 100.672908) (mid 169.50053 99.4575) (end 168.997092 98.242092) (width 0.4) (layer "F.Cu") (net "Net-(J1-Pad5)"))
 (arc (start 168.979542 98.224542) (mid 167.922209 97.518064) (end 166.675 97.27) (width 0.4) (layer "F.Cu") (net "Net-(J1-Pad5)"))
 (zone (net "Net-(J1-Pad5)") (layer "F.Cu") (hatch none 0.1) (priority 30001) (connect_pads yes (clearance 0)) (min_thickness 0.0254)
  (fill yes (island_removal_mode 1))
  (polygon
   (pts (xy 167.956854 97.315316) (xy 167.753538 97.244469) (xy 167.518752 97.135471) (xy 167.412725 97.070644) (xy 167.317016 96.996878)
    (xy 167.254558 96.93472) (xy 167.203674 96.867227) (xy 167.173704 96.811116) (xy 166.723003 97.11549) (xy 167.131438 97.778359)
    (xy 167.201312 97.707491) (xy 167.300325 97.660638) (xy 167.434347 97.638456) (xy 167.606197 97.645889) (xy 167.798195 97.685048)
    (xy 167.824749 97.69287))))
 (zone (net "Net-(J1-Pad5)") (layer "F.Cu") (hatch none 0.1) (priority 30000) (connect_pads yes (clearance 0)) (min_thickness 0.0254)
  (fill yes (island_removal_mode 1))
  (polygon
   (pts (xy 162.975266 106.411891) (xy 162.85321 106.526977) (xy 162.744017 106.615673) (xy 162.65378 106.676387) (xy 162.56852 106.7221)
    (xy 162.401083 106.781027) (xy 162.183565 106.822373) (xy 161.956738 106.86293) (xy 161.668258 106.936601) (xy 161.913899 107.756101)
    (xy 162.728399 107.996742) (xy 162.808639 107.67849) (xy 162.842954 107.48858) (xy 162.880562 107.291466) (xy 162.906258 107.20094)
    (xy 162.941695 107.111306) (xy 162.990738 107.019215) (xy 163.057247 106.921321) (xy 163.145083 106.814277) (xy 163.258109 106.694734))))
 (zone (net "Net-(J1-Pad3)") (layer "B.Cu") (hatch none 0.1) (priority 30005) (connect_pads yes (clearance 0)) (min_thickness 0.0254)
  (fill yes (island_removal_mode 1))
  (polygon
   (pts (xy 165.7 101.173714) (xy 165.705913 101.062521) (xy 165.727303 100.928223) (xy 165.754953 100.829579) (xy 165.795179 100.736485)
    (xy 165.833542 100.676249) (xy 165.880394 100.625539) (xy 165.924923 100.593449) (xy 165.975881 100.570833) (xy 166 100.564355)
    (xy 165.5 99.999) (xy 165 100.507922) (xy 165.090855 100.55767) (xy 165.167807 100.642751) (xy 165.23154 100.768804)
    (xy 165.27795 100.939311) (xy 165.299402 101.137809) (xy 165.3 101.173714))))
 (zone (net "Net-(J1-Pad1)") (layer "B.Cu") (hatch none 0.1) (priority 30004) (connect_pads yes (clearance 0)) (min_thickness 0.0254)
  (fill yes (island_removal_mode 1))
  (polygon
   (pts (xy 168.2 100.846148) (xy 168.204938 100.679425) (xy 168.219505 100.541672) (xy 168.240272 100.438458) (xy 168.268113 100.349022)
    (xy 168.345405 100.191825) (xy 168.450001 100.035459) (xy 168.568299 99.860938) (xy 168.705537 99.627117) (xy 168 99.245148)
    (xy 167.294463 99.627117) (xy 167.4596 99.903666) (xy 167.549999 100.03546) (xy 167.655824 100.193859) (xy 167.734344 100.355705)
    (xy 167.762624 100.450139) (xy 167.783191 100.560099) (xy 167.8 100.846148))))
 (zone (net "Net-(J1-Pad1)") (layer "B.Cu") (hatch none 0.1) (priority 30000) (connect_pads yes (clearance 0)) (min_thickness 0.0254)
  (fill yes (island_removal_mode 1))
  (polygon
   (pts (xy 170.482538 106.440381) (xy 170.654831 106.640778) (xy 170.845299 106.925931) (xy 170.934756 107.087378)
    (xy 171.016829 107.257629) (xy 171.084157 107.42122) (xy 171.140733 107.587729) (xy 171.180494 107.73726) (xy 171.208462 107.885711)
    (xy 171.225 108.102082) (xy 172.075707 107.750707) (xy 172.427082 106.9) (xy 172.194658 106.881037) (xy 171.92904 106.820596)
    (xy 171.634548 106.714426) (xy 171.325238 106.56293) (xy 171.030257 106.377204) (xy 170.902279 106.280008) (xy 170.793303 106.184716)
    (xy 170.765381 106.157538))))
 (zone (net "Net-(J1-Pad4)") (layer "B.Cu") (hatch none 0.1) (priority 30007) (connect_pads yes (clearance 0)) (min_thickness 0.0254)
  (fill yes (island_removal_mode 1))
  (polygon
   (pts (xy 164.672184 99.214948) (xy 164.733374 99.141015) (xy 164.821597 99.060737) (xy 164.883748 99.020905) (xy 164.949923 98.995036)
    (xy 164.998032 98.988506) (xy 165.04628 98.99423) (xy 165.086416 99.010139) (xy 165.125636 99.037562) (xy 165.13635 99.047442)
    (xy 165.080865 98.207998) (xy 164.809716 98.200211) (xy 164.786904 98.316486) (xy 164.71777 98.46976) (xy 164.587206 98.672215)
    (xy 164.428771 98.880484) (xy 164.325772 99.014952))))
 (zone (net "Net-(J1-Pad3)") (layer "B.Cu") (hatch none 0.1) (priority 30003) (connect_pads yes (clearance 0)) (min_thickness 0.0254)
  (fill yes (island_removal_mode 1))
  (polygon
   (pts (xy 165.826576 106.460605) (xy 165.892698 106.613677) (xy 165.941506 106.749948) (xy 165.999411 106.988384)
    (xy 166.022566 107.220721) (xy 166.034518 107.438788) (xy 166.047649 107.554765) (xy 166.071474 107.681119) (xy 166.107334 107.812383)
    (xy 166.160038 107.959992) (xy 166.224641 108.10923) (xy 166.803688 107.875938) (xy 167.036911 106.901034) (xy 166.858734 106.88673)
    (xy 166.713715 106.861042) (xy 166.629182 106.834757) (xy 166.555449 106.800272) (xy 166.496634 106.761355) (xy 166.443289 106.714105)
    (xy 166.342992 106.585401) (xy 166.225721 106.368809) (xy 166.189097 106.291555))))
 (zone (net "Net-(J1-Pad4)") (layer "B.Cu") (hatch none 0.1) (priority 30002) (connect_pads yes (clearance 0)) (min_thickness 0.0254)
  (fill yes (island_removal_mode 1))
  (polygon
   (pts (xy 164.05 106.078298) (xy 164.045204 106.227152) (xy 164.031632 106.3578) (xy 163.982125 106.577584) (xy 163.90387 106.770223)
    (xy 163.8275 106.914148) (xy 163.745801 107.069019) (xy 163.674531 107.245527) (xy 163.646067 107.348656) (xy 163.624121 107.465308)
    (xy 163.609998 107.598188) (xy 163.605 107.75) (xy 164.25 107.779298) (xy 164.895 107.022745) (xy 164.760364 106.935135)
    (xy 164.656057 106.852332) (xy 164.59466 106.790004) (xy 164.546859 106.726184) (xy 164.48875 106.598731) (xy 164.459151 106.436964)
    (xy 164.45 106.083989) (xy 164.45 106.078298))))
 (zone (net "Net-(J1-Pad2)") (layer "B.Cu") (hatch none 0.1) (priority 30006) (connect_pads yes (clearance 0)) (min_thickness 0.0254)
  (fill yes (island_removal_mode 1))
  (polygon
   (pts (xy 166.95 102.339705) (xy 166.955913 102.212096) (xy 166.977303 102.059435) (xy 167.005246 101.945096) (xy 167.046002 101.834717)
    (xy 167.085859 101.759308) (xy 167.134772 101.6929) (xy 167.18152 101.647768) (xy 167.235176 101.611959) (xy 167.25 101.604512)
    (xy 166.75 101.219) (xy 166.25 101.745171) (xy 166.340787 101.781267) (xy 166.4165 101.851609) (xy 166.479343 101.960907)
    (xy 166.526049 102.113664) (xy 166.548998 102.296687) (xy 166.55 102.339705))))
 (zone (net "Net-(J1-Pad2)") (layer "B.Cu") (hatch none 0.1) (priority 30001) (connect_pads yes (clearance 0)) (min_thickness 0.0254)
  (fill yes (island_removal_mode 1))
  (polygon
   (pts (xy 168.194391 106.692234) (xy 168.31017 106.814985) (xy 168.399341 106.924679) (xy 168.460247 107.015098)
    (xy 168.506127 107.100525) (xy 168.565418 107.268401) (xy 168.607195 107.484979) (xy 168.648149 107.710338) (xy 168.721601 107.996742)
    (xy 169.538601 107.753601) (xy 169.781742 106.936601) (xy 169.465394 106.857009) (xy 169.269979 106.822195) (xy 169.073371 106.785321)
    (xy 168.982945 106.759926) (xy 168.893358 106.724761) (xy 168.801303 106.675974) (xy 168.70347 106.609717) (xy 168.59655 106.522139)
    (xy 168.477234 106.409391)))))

